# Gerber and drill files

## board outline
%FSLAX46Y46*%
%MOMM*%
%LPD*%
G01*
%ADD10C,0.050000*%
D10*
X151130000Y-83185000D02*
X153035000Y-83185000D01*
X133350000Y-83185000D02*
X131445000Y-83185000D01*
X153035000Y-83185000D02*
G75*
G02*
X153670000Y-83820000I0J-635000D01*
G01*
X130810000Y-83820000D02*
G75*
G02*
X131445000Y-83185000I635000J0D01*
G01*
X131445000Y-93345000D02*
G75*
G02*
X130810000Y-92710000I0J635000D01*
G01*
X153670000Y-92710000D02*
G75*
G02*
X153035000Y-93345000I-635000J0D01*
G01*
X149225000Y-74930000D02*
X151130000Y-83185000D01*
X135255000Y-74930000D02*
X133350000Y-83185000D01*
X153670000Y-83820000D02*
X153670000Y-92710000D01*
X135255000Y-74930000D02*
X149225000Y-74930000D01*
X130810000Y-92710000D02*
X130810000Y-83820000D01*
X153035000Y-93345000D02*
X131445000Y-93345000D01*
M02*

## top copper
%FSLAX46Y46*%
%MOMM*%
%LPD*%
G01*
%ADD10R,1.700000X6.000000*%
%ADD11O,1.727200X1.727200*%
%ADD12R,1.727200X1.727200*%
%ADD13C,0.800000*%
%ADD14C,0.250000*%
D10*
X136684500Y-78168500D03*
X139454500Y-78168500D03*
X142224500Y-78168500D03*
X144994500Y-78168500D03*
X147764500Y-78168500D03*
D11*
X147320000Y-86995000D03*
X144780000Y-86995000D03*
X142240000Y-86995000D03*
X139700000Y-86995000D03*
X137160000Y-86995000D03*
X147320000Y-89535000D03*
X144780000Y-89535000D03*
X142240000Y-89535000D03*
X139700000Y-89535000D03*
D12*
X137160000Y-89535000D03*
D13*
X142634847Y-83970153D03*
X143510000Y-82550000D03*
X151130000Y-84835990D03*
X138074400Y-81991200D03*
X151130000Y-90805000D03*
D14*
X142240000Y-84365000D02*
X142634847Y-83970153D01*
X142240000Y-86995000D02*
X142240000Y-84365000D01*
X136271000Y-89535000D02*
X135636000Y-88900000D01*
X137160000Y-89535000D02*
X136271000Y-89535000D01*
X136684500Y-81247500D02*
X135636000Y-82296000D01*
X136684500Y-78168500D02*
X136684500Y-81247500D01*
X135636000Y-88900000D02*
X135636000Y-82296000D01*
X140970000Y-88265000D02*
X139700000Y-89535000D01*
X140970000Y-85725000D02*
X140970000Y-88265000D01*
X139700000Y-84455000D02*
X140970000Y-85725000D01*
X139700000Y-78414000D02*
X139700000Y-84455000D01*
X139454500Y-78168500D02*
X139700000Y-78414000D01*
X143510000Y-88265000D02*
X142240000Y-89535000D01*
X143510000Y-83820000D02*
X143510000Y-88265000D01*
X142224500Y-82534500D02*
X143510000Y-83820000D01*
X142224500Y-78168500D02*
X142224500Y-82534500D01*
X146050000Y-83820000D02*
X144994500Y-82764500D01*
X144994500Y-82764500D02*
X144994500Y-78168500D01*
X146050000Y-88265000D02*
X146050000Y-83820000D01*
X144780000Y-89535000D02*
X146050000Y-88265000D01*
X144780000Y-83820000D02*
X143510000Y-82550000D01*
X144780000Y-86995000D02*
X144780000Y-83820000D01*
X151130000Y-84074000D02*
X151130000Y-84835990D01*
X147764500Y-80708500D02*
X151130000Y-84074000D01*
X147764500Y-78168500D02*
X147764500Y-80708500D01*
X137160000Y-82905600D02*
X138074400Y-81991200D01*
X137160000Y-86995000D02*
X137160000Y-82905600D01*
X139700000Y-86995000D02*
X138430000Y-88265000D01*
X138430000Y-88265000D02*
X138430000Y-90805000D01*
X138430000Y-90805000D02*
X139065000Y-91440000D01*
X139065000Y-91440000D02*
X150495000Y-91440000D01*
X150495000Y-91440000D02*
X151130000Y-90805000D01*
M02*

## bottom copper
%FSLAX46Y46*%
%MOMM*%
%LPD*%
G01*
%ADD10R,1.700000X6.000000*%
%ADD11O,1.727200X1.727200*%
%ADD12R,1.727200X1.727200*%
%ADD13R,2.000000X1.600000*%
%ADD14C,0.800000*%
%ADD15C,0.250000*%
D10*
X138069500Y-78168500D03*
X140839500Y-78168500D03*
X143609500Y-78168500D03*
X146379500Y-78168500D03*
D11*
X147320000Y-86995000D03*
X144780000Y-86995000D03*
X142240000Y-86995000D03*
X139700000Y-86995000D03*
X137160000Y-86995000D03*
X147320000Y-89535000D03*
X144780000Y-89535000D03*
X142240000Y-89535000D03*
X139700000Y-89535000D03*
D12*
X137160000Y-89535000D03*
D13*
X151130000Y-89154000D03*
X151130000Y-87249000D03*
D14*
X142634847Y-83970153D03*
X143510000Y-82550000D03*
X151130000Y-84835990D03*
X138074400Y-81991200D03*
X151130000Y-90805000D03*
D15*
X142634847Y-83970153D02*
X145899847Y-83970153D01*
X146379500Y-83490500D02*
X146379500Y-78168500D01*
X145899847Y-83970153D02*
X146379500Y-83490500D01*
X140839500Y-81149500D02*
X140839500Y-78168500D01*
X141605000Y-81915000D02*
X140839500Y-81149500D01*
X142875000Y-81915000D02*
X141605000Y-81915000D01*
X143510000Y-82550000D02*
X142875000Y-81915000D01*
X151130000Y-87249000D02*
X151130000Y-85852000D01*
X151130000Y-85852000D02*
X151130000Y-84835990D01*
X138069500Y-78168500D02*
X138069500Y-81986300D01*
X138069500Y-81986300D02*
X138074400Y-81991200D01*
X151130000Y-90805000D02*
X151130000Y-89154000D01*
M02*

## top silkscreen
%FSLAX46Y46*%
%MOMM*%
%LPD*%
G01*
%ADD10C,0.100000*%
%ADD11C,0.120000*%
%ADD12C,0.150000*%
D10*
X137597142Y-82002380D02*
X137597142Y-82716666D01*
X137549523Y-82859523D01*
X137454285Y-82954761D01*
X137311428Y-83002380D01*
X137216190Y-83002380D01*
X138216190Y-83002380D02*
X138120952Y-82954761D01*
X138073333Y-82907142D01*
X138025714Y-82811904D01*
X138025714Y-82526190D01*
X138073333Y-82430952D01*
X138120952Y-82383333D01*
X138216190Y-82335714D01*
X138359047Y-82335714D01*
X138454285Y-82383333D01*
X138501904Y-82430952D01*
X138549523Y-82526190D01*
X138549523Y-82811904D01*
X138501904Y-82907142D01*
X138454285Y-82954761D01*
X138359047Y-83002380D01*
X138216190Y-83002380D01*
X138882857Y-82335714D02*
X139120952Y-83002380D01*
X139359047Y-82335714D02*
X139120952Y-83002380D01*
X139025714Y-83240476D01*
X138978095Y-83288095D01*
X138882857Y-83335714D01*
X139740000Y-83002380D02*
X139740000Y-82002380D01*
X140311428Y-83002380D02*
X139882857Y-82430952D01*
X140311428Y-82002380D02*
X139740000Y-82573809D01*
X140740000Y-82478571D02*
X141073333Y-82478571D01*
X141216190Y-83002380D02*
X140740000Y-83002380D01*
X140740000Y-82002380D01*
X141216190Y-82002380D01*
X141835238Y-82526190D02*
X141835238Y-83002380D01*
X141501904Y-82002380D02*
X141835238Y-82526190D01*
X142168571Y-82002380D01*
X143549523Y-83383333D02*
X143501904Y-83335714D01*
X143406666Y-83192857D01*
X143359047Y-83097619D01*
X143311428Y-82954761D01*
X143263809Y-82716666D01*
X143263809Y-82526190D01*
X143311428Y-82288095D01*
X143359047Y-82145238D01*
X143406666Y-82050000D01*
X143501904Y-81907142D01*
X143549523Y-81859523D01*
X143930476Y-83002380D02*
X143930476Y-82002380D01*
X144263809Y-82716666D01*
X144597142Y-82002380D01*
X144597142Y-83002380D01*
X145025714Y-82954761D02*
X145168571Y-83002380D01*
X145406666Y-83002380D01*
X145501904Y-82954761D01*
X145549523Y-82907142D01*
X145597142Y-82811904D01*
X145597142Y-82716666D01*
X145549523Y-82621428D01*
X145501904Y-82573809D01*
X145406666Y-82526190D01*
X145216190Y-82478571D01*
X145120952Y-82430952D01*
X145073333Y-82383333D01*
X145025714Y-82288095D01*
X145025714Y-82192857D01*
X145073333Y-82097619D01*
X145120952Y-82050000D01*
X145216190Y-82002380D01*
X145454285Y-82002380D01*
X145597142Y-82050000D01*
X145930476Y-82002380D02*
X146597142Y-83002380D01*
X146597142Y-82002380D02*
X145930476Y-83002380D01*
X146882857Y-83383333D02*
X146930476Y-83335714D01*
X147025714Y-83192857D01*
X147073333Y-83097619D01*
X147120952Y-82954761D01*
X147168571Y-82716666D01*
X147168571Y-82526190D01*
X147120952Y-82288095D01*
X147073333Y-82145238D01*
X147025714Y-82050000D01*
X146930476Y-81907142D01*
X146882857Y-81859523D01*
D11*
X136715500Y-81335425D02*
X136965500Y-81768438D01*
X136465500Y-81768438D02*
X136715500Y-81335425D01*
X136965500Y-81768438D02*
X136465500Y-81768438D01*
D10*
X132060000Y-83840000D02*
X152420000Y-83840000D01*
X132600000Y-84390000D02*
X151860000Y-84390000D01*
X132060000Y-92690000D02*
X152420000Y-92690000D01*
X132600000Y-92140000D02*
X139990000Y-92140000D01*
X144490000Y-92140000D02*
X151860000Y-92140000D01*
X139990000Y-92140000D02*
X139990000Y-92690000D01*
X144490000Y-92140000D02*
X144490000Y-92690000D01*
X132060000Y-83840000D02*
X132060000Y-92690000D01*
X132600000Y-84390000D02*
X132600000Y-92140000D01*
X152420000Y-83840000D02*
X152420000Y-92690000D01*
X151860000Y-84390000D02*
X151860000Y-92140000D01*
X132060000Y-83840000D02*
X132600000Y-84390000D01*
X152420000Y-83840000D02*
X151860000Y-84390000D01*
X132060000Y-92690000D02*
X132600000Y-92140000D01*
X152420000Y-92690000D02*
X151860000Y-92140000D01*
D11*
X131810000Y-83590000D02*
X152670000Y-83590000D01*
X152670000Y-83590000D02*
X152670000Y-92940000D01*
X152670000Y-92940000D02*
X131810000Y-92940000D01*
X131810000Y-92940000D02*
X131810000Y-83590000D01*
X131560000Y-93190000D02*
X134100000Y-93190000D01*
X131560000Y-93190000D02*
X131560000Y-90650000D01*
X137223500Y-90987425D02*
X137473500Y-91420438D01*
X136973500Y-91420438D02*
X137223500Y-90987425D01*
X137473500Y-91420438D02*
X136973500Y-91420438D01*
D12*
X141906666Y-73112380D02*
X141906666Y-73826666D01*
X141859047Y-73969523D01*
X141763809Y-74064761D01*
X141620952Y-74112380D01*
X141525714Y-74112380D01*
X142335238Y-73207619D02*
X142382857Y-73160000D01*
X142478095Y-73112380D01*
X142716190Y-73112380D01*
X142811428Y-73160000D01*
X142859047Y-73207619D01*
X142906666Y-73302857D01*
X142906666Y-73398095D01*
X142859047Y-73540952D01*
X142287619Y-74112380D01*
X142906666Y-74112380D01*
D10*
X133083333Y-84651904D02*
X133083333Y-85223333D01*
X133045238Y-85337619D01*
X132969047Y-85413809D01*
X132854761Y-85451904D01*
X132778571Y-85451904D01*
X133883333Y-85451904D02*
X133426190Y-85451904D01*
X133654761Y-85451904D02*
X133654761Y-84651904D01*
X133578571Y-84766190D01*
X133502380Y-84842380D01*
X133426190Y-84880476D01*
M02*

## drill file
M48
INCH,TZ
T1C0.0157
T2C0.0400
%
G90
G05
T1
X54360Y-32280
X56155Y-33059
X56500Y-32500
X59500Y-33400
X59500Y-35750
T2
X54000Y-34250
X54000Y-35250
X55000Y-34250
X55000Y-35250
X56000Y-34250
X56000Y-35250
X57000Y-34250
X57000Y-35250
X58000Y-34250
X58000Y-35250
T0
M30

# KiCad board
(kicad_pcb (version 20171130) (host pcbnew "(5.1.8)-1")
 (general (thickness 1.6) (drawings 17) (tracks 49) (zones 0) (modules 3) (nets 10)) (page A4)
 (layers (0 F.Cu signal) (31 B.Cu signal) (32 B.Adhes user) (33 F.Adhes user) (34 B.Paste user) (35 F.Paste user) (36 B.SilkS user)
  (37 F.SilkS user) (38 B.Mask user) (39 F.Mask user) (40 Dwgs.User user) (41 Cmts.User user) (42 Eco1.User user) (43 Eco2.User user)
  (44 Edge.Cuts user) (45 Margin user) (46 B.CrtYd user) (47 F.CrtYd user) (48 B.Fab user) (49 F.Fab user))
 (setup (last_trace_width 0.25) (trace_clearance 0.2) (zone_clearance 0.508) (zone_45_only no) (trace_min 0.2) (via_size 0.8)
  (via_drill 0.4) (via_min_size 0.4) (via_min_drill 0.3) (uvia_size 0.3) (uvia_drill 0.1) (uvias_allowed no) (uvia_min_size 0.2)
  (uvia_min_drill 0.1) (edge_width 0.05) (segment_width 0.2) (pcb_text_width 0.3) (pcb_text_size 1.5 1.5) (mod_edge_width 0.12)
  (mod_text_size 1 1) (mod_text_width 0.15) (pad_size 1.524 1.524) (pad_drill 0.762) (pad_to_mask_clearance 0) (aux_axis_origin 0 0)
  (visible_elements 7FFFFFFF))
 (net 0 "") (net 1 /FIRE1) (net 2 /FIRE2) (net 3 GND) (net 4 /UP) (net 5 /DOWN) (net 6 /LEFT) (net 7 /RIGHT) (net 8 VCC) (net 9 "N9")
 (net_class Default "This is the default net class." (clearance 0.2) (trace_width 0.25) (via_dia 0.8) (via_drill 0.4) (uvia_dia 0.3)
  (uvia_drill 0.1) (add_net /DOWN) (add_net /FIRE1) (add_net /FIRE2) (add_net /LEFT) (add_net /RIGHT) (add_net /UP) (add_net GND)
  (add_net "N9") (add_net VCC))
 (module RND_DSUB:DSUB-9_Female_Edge (layer F.Cu) (at 142.24 78.105)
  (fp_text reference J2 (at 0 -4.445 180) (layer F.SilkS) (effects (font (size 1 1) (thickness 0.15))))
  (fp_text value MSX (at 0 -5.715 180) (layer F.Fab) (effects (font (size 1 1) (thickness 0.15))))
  (fp_line (start -5.5245 3.230425) (end -5.2745 3.663438) (layer F.SilkS) (width 0.12))
  (fp_line (start -5.7745 3.663438) (end -5.5245 3.230425) (layer F.SilkS) (width 0.12))
  (fp_line (start -5.2745 3.663438) (end -5.7745 3.663438) (layer F.SilkS) (width 0.12))
  (pad 6 smd rect (at -4.1705 0.0635 180) (size 1.7 6) (layers B.Cu B.Paste B.Mask) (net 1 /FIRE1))
  (pad 7 smd rect (at -1.4005 0.0635 180) (size 1.7 6) (layers B.Cu B.Paste B.Mask) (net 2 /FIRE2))
  (pad 8 smd rect (at 1.3695 0.0635 180) (size 1.7 6) (layers B.Cu B.Paste B.Mask))
  (pad 9 smd rect (at 4.1395 0.0635 180) (size 1.7 6) (layers B.Cu B.Paste B.Mask) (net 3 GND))
  (pad 1 smd rect (at -5.5555 0.0635 180) (size 1.7 6) (layers F.Cu F.Paste F.Mask) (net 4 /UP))
  (pad 2 smd rect (at -2.7855 0.0635 180) (size 1.7 6) (layers F.Cu F.Paste F.Mask) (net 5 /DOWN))
  (pad 3 smd rect (at -0.0155 0.0635 180) (size 1.7 6) (layers F.Cu F.Paste F.Mask) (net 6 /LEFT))
  (pad 4 smd rect (at 2.7545 0.0635 180) (size 1.7 6) (layers F.Cu F.Paste F.Mask) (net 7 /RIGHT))
  (pad 5 smd rect (at 5.5245 0.0635 180) (size 1.7 6) (layers F.Cu F.Paste F.Mask) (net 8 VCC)))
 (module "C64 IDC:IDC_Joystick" (layer F.Cu) (at 137.16 89.535 90)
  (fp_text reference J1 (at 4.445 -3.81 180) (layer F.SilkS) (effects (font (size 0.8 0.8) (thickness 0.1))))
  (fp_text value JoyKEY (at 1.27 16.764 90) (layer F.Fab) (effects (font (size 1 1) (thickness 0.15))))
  (fp_line (start 5.695 -5.1) (end 5.695 15.26) (layer F.SilkS) (width 0.1))
  (fp_line (start 5.145 -4.56) (end 5.145 14.7) (layer F.SilkS) (width 0.1))
  (fp_line (start -3.155 -5.1) (end -3.155 15.26) (layer F.SilkS) (width 0.1))
  (fp_line (start -2.605 -4.56) (end -2.605 2.83) (layer F.SilkS) (width 0.1))
  (fp_line (start -2.605 7.33) (end -2.605 14.7) (layer F.SilkS) (width 0.1))
  (fp_line (start -2.605 2.83) (end -3.155 2.83) (layer F.SilkS) (width 0.1))
  (fp_line (start -2.605 7.33) (end -3.155 7.33) (layer F.SilkS) (width 0.1))
  (fp_line (start 5.695 -5.1) (end -3.155 -5.1) (layer F.SilkS) (width 0.1))
  (fp_line (start 5.145 -4.56) (end -2.605 -4.56) (layer F.SilkS) (width 0.1))
  (fp_line (start 5.695 15.26) (end -3.155 15.26) (layer F.SilkS) (width 0.1))
  (fp_line (start 5.145 14.7) (end -2.605 14.7) (layer F.SilkS) (width 0.1))
  (fp_line (start 5.695 -5.1) (end 5.145 -4.56) (layer F.SilkS) (width 0.1))
  (fp_line (start 5.695 15.26) (end 5.145 14.7) (layer F.SilkS) (width 0.1))
  (fp_line (start -3.155 -5.1) (end -2.605 -4.56) (layer F.SilkS) (width 0.1))
  (fp_line (start -3.155 15.26) (end -2.605 14.7) (layer F.SilkS) (width 0.1))
  (fp_line (start 5.945 -5.35) (end 5.945 15.51) (layer F.SilkS) (width 0.12))
  (fp_line (start 5.945 15.51) (end -3.405 15.51) (layer F.SilkS) (width 0.12))
  (fp_line (start -3.405 15.51) (end -3.405 -5.35) (layer F.SilkS) (width 0.12))
  (fp_line (start -3.405 -5.35) (end 5.945 -5.35) (layer F.SilkS) (width 0.12))
  (fp_line (start -3.655 -5.6) (end -3.655 -3.06) (layer F.SilkS) (width 0.12))
  (fp_line (start -3.655 -5.6) (end -1.115 -5.6) (layer F.SilkS) (width 0.12))
  (fp_line (start -1.452425 0.0635) (end -1.885438 0.3135) (layer F.SilkS) (width 0.12))
  (fp_line (start -1.885438 -0.1865) (end -1.452425 0.0635) (layer F.SilkS) (width 0.12))
  (fp_line (start -1.885438 0.3135) (end -1.885438 -0.1865) (layer F.SilkS) (width 0.12))
  (pad 10 thru_hole oval (at 2.54 10.16 90) (size 1.7272 1.7272) (drill 1.016) (layers *.Cu *.Mask))
  (pad 9 thru_hole oval (at 2.54 7.62 90) (size 1.7272 1.7272) (drill 1.016) (layers *.Cu *.Mask) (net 2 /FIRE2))
  (pad 8 thru_hole oval (at 2.54 5.08 90) (size 1.7272 1.7272) (drill 1.016) (layers *.Cu *.Mask) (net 3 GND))
  (pad 7 thru_hole oval (at 2.54 2.54 90) (size 1.7272 1.7272) (drill 1.016) (layers *.Cu *.Mask) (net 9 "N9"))
  (pad 6 thru_hole oval (at 2.54 0 90) (size 1.7272 1.7272) (drill 1.016) (layers *.Cu *.Mask) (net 1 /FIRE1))
  (pad 5 thru_hole oval (at 0 10.16 90) (size 1.7272 1.7272) (drill 1.016) (layers *.Cu *.Mask))
  (pad 4 thru_hole oval (at 0 7.62 90) (size 1.7272 1.7272) (drill 1.016) (layers *.Cu *.Mask) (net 7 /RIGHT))
  (pad 3 thru_hole oval (at 0 5.08 90) (size 1.7272 1.7272) (drill 1.016) (layers *.Cu *.Mask) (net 6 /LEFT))
  (pad 2 thru_hole oval (at 0 2.54 90) (size 1.7272 1.7272) (drill 1.016) (layers *.Cu *.Mask) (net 5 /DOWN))
  (pad 1 thru_hole rect (at 0 0 90) (size 1.7272 1.7272) (drill 1.016) (layers *.Cu *.Mask) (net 4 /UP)))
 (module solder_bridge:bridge (layer B.Cu) (at 151.13 89.154)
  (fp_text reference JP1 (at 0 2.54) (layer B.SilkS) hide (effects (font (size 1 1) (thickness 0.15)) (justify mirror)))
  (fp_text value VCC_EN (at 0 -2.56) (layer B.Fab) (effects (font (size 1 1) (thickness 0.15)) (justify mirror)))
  (pad 1 smd rect (at 0 0) (size 2 1.6) (layers B.Cu B.Paste B.Mask) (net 9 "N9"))
  (pad 2 smd rect (at 0 -1.905) (size 2 1.6) (layers B.Cu B.Paste B.Mask) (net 8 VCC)))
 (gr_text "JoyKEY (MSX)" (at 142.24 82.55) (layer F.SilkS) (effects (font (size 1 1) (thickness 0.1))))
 (gr_line (start 151.13 83.185) (end 153.035 83.185) (layer Edge.Cuts) (width 0.05))
 (gr_line (start 133.35 83.185) (end 131.445 83.185) (layer Edge.Cuts) (width 0.05))
 (gr_arc (start 153.035 83.82) (end 153.67 83.82) (angle -90) (layer Edge.Cuts) (width 0.05))
 (gr_arc (start 131.445 83.82) (end 131.445 83.185) (angle -90) (layer Edge.Cuts) (width 0.05))
 (gr_arc (start 131.445 92.71) (end 130.81 92.71) (angle -90) (layer Edge.Cuts) (width 0.05))
 (gr_arc (start 153.035 92.71) (end 153.035 93.345) (angle -90) (layer Edge.Cuts) (width 0.05))
 (gr_line (start 149.225 74.93) (end 151.13 83.185) (layer Edge.Cuts) (width 0.05))
 (gr_line (start 135.255 74.93) (end 133.35 83.185) (layer Edge.Cuts) (width 0.05))
 (gr_line (start 153.67 83.82) (end 153.67 92.71) (layer Edge.Cuts) (width 0.05))
 (gr_line (start 135.255 74.93) (end 149.225 74.93) (layer Edge.Cuts) (width 0.05))
 (gr_line (start 130.81 92.71) (end 130.81 83.82) (layer Edge.Cuts) (width 0.05))
 (gr_line (start 153.035 93.345) (end 131.445 93.345) (layer Edge.Cuts) (width 0.05))
 (via (at 142.634847 83.970153) (size 0.8) (drill 0.4) (layers F.Cu B.Cu) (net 3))
 (segment (start 142.24 84.365) (end 142.634847 83.970153) (width 0.25) (layer F.Cu) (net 3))
 (segment (start 142.24 86.995) (end 142.24 84.365) (width 0.25) (layer F.Cu) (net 3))
 (segment (start 142.634847 83.970153) (end 145.899847 83.970153) (width 0.25) (layer B.Cu) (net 3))
 (segment (start 146.3795 83.4905) (end 146.3795 78.1685) (width 0.25) (layer B.Cu) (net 3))
 (segment (start 145.899847 83.970153) (end 146.3795 83.4905) (width 0.25) (layer B.Cu) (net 3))
 (segment (start 136.271 89.535) (end 135.636 88.9) (width 0.25) (layer F.Cu) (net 4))
 (segment (start 137.16 89.535) (end 136.271 89.535) (width 0.25) (layer F.Cu) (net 4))
 (segment (start 136.6845 81.2475) (end 135.636 82.296) (width 0.25) (layer F.Cu) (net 4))
 (segment (start 136.6845 78.1685) (end 136.6845 81.2475) (width 0.25) (layer F.Cu) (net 4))
 (segment (start 135.636 88.9) (end 135.636 82.296) (width 0.25) (layer F.Cu) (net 4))
 (segment (start 140.97 88.265) (end 139.7 89.535) (width 0.25) (layer F.Cu) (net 5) (status 20))
 (segment (start 140.97 85.725) (end 140.97 88.265) (width 0.25) (layer F.Cu) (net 5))
 (segment (start 139.7 84.455) (end 140.97 85.725) (width 0.25) (layer F.Cu) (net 5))
 (segment (start 139.7 78.414) (end 139.7 84.455) (width 0.25) (layer F.Cu) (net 5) (status 10))
 (segment (start 139.4545 78.1685) (end 139.7 78.414) (width 0.25) (layer F.Cu) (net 5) (status 30))
 (segment (start 143.51 88.265) (end 142.24 89.535) (width 0.25) (layer F.Cu) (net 6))
 (segment (start 143.51 83.82) (end 143.51 88.265) (width 0.25) (layer F.Cu) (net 6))
 (segment (start 142.2245 82.5345) (end 143.51 83.82) (width 0.25) (layer F.Cu) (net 6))
 (segment (start 142.2245 78.1685) (end 142.2245 82.5345) (width 0.25) (layer F.Cu) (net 6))
 (segment (start 146.05 83.82) (end 144.9945 82.7645) (width 0.25) (layer F.Cu) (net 7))
 (segment (start 144.9945 82.7645) (end 144.9945 78.1685) (width 0.25) (layer F.Cu) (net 7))
 (segment (start 146.05 88.265) (end 146.05 83.82) (width 0.25) (layer F.Cu) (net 7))
 (segment (start 144.78 89.535) (end 146.05 88.265) (width 0.25) (layer F.Cu) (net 7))
 (via (at 143.51 82.55) (size 0.8) (drill 0.4) (layers F.Cu B.Cu) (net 2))
 (segment (start 140.8395 81.1495) (end 140.8395 78.1685) (width 0.25) (layer B.Cu) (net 2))
 (segment (start 141.605 81.915) (end 140.8395 81.1495) (width 0.25) (layer B.Cu) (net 2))
 (segment (start 142.875 81.915) (end 141.605 81.915) (width 0.25) (layer B.Cu) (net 2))
 (segment (start 143.51 82.55) (end 142.875 81.915) (width 0.25) (layer B.Cu) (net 2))
 (segment (start 144.78 83.82) (end 143.51 82.55) (width 0.25) (layer F.Cu) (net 2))
 (segment (start 144.78 86.995) (end 144.78 83.82) (width 0.25) (layer F.Cu) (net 2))
 (segment (start 151.13 87.249) (end 151.13 85.852) (width 0.25) (layer B.Cu) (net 8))
 (segment (start 151.13 85.852) (end 151.13 84.83599) (width 0.25) (layer B.Cu) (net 8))
 (via (at 151.13 84.83599) (size 0.8) (drill 0.4) (layers F.Cu B.Cu) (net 8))
 (segment (start 151.13 84.074) (end 151.13 84.83599) (width 0.25) (layer F.Cu) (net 8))
 (segment (start 147.7645 80.7085) (end 151.13 84.074) (width 0.25) (layer F.Cu) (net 8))
 (segment (start 147.7645 78.1685) (end 147.7645 80.7085) (width 0.25) (layer F.Cu) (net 8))
 (segment (start 138.0695 78.1685) (end 138.0695 81.9863) (width 0.25) (layer B.Cu) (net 1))
 (segment (start 138.0695 81.9863) (end 138.0744 81.9912) (width 0.25) (layer B.Cu) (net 1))
 (segment (start 137.16 82.9056) (end 138.0744 81.9912) (width 0.25) (layer F.Cu) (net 1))
 (segment (start 137.16 86.995) (end 137.16 82.9056) (width 0.25) (layer F.Cu) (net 1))
 (via (at 138.0744 81.9912) (size 0.8) (drill 0.4) (layers F.Cu B.Cu) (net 1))
 (segment (start 139.7 86.995) (end 138.43 88.265) (width 0.25) (layer F.Cu) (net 9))
 (segment (start 138.43 88.265) (end 138.43 90.805) (width 0.25) (layer F.Cu) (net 9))
 (segment (start 138.43 90.805) (end 139.065 91.44) (width 0.25) (layer F.Cu) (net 9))
 (segment (start 139.065 91.44) (end 150.495 91.44) (width 0.25) (layer F.Cu) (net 9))
 (via (at 151.13 90.805) (size 0.8) (drill 0.4) (layers F.Cu B.Cu) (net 9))
 (segment (start 150.495 91.44) (end 151.13 90.805) (width 0.25) (layer F.Cu) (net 9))
 (segment (start 151.13 90.805) (end 151.13 89.154) (width 0.25) (layer B.Cu) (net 9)))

